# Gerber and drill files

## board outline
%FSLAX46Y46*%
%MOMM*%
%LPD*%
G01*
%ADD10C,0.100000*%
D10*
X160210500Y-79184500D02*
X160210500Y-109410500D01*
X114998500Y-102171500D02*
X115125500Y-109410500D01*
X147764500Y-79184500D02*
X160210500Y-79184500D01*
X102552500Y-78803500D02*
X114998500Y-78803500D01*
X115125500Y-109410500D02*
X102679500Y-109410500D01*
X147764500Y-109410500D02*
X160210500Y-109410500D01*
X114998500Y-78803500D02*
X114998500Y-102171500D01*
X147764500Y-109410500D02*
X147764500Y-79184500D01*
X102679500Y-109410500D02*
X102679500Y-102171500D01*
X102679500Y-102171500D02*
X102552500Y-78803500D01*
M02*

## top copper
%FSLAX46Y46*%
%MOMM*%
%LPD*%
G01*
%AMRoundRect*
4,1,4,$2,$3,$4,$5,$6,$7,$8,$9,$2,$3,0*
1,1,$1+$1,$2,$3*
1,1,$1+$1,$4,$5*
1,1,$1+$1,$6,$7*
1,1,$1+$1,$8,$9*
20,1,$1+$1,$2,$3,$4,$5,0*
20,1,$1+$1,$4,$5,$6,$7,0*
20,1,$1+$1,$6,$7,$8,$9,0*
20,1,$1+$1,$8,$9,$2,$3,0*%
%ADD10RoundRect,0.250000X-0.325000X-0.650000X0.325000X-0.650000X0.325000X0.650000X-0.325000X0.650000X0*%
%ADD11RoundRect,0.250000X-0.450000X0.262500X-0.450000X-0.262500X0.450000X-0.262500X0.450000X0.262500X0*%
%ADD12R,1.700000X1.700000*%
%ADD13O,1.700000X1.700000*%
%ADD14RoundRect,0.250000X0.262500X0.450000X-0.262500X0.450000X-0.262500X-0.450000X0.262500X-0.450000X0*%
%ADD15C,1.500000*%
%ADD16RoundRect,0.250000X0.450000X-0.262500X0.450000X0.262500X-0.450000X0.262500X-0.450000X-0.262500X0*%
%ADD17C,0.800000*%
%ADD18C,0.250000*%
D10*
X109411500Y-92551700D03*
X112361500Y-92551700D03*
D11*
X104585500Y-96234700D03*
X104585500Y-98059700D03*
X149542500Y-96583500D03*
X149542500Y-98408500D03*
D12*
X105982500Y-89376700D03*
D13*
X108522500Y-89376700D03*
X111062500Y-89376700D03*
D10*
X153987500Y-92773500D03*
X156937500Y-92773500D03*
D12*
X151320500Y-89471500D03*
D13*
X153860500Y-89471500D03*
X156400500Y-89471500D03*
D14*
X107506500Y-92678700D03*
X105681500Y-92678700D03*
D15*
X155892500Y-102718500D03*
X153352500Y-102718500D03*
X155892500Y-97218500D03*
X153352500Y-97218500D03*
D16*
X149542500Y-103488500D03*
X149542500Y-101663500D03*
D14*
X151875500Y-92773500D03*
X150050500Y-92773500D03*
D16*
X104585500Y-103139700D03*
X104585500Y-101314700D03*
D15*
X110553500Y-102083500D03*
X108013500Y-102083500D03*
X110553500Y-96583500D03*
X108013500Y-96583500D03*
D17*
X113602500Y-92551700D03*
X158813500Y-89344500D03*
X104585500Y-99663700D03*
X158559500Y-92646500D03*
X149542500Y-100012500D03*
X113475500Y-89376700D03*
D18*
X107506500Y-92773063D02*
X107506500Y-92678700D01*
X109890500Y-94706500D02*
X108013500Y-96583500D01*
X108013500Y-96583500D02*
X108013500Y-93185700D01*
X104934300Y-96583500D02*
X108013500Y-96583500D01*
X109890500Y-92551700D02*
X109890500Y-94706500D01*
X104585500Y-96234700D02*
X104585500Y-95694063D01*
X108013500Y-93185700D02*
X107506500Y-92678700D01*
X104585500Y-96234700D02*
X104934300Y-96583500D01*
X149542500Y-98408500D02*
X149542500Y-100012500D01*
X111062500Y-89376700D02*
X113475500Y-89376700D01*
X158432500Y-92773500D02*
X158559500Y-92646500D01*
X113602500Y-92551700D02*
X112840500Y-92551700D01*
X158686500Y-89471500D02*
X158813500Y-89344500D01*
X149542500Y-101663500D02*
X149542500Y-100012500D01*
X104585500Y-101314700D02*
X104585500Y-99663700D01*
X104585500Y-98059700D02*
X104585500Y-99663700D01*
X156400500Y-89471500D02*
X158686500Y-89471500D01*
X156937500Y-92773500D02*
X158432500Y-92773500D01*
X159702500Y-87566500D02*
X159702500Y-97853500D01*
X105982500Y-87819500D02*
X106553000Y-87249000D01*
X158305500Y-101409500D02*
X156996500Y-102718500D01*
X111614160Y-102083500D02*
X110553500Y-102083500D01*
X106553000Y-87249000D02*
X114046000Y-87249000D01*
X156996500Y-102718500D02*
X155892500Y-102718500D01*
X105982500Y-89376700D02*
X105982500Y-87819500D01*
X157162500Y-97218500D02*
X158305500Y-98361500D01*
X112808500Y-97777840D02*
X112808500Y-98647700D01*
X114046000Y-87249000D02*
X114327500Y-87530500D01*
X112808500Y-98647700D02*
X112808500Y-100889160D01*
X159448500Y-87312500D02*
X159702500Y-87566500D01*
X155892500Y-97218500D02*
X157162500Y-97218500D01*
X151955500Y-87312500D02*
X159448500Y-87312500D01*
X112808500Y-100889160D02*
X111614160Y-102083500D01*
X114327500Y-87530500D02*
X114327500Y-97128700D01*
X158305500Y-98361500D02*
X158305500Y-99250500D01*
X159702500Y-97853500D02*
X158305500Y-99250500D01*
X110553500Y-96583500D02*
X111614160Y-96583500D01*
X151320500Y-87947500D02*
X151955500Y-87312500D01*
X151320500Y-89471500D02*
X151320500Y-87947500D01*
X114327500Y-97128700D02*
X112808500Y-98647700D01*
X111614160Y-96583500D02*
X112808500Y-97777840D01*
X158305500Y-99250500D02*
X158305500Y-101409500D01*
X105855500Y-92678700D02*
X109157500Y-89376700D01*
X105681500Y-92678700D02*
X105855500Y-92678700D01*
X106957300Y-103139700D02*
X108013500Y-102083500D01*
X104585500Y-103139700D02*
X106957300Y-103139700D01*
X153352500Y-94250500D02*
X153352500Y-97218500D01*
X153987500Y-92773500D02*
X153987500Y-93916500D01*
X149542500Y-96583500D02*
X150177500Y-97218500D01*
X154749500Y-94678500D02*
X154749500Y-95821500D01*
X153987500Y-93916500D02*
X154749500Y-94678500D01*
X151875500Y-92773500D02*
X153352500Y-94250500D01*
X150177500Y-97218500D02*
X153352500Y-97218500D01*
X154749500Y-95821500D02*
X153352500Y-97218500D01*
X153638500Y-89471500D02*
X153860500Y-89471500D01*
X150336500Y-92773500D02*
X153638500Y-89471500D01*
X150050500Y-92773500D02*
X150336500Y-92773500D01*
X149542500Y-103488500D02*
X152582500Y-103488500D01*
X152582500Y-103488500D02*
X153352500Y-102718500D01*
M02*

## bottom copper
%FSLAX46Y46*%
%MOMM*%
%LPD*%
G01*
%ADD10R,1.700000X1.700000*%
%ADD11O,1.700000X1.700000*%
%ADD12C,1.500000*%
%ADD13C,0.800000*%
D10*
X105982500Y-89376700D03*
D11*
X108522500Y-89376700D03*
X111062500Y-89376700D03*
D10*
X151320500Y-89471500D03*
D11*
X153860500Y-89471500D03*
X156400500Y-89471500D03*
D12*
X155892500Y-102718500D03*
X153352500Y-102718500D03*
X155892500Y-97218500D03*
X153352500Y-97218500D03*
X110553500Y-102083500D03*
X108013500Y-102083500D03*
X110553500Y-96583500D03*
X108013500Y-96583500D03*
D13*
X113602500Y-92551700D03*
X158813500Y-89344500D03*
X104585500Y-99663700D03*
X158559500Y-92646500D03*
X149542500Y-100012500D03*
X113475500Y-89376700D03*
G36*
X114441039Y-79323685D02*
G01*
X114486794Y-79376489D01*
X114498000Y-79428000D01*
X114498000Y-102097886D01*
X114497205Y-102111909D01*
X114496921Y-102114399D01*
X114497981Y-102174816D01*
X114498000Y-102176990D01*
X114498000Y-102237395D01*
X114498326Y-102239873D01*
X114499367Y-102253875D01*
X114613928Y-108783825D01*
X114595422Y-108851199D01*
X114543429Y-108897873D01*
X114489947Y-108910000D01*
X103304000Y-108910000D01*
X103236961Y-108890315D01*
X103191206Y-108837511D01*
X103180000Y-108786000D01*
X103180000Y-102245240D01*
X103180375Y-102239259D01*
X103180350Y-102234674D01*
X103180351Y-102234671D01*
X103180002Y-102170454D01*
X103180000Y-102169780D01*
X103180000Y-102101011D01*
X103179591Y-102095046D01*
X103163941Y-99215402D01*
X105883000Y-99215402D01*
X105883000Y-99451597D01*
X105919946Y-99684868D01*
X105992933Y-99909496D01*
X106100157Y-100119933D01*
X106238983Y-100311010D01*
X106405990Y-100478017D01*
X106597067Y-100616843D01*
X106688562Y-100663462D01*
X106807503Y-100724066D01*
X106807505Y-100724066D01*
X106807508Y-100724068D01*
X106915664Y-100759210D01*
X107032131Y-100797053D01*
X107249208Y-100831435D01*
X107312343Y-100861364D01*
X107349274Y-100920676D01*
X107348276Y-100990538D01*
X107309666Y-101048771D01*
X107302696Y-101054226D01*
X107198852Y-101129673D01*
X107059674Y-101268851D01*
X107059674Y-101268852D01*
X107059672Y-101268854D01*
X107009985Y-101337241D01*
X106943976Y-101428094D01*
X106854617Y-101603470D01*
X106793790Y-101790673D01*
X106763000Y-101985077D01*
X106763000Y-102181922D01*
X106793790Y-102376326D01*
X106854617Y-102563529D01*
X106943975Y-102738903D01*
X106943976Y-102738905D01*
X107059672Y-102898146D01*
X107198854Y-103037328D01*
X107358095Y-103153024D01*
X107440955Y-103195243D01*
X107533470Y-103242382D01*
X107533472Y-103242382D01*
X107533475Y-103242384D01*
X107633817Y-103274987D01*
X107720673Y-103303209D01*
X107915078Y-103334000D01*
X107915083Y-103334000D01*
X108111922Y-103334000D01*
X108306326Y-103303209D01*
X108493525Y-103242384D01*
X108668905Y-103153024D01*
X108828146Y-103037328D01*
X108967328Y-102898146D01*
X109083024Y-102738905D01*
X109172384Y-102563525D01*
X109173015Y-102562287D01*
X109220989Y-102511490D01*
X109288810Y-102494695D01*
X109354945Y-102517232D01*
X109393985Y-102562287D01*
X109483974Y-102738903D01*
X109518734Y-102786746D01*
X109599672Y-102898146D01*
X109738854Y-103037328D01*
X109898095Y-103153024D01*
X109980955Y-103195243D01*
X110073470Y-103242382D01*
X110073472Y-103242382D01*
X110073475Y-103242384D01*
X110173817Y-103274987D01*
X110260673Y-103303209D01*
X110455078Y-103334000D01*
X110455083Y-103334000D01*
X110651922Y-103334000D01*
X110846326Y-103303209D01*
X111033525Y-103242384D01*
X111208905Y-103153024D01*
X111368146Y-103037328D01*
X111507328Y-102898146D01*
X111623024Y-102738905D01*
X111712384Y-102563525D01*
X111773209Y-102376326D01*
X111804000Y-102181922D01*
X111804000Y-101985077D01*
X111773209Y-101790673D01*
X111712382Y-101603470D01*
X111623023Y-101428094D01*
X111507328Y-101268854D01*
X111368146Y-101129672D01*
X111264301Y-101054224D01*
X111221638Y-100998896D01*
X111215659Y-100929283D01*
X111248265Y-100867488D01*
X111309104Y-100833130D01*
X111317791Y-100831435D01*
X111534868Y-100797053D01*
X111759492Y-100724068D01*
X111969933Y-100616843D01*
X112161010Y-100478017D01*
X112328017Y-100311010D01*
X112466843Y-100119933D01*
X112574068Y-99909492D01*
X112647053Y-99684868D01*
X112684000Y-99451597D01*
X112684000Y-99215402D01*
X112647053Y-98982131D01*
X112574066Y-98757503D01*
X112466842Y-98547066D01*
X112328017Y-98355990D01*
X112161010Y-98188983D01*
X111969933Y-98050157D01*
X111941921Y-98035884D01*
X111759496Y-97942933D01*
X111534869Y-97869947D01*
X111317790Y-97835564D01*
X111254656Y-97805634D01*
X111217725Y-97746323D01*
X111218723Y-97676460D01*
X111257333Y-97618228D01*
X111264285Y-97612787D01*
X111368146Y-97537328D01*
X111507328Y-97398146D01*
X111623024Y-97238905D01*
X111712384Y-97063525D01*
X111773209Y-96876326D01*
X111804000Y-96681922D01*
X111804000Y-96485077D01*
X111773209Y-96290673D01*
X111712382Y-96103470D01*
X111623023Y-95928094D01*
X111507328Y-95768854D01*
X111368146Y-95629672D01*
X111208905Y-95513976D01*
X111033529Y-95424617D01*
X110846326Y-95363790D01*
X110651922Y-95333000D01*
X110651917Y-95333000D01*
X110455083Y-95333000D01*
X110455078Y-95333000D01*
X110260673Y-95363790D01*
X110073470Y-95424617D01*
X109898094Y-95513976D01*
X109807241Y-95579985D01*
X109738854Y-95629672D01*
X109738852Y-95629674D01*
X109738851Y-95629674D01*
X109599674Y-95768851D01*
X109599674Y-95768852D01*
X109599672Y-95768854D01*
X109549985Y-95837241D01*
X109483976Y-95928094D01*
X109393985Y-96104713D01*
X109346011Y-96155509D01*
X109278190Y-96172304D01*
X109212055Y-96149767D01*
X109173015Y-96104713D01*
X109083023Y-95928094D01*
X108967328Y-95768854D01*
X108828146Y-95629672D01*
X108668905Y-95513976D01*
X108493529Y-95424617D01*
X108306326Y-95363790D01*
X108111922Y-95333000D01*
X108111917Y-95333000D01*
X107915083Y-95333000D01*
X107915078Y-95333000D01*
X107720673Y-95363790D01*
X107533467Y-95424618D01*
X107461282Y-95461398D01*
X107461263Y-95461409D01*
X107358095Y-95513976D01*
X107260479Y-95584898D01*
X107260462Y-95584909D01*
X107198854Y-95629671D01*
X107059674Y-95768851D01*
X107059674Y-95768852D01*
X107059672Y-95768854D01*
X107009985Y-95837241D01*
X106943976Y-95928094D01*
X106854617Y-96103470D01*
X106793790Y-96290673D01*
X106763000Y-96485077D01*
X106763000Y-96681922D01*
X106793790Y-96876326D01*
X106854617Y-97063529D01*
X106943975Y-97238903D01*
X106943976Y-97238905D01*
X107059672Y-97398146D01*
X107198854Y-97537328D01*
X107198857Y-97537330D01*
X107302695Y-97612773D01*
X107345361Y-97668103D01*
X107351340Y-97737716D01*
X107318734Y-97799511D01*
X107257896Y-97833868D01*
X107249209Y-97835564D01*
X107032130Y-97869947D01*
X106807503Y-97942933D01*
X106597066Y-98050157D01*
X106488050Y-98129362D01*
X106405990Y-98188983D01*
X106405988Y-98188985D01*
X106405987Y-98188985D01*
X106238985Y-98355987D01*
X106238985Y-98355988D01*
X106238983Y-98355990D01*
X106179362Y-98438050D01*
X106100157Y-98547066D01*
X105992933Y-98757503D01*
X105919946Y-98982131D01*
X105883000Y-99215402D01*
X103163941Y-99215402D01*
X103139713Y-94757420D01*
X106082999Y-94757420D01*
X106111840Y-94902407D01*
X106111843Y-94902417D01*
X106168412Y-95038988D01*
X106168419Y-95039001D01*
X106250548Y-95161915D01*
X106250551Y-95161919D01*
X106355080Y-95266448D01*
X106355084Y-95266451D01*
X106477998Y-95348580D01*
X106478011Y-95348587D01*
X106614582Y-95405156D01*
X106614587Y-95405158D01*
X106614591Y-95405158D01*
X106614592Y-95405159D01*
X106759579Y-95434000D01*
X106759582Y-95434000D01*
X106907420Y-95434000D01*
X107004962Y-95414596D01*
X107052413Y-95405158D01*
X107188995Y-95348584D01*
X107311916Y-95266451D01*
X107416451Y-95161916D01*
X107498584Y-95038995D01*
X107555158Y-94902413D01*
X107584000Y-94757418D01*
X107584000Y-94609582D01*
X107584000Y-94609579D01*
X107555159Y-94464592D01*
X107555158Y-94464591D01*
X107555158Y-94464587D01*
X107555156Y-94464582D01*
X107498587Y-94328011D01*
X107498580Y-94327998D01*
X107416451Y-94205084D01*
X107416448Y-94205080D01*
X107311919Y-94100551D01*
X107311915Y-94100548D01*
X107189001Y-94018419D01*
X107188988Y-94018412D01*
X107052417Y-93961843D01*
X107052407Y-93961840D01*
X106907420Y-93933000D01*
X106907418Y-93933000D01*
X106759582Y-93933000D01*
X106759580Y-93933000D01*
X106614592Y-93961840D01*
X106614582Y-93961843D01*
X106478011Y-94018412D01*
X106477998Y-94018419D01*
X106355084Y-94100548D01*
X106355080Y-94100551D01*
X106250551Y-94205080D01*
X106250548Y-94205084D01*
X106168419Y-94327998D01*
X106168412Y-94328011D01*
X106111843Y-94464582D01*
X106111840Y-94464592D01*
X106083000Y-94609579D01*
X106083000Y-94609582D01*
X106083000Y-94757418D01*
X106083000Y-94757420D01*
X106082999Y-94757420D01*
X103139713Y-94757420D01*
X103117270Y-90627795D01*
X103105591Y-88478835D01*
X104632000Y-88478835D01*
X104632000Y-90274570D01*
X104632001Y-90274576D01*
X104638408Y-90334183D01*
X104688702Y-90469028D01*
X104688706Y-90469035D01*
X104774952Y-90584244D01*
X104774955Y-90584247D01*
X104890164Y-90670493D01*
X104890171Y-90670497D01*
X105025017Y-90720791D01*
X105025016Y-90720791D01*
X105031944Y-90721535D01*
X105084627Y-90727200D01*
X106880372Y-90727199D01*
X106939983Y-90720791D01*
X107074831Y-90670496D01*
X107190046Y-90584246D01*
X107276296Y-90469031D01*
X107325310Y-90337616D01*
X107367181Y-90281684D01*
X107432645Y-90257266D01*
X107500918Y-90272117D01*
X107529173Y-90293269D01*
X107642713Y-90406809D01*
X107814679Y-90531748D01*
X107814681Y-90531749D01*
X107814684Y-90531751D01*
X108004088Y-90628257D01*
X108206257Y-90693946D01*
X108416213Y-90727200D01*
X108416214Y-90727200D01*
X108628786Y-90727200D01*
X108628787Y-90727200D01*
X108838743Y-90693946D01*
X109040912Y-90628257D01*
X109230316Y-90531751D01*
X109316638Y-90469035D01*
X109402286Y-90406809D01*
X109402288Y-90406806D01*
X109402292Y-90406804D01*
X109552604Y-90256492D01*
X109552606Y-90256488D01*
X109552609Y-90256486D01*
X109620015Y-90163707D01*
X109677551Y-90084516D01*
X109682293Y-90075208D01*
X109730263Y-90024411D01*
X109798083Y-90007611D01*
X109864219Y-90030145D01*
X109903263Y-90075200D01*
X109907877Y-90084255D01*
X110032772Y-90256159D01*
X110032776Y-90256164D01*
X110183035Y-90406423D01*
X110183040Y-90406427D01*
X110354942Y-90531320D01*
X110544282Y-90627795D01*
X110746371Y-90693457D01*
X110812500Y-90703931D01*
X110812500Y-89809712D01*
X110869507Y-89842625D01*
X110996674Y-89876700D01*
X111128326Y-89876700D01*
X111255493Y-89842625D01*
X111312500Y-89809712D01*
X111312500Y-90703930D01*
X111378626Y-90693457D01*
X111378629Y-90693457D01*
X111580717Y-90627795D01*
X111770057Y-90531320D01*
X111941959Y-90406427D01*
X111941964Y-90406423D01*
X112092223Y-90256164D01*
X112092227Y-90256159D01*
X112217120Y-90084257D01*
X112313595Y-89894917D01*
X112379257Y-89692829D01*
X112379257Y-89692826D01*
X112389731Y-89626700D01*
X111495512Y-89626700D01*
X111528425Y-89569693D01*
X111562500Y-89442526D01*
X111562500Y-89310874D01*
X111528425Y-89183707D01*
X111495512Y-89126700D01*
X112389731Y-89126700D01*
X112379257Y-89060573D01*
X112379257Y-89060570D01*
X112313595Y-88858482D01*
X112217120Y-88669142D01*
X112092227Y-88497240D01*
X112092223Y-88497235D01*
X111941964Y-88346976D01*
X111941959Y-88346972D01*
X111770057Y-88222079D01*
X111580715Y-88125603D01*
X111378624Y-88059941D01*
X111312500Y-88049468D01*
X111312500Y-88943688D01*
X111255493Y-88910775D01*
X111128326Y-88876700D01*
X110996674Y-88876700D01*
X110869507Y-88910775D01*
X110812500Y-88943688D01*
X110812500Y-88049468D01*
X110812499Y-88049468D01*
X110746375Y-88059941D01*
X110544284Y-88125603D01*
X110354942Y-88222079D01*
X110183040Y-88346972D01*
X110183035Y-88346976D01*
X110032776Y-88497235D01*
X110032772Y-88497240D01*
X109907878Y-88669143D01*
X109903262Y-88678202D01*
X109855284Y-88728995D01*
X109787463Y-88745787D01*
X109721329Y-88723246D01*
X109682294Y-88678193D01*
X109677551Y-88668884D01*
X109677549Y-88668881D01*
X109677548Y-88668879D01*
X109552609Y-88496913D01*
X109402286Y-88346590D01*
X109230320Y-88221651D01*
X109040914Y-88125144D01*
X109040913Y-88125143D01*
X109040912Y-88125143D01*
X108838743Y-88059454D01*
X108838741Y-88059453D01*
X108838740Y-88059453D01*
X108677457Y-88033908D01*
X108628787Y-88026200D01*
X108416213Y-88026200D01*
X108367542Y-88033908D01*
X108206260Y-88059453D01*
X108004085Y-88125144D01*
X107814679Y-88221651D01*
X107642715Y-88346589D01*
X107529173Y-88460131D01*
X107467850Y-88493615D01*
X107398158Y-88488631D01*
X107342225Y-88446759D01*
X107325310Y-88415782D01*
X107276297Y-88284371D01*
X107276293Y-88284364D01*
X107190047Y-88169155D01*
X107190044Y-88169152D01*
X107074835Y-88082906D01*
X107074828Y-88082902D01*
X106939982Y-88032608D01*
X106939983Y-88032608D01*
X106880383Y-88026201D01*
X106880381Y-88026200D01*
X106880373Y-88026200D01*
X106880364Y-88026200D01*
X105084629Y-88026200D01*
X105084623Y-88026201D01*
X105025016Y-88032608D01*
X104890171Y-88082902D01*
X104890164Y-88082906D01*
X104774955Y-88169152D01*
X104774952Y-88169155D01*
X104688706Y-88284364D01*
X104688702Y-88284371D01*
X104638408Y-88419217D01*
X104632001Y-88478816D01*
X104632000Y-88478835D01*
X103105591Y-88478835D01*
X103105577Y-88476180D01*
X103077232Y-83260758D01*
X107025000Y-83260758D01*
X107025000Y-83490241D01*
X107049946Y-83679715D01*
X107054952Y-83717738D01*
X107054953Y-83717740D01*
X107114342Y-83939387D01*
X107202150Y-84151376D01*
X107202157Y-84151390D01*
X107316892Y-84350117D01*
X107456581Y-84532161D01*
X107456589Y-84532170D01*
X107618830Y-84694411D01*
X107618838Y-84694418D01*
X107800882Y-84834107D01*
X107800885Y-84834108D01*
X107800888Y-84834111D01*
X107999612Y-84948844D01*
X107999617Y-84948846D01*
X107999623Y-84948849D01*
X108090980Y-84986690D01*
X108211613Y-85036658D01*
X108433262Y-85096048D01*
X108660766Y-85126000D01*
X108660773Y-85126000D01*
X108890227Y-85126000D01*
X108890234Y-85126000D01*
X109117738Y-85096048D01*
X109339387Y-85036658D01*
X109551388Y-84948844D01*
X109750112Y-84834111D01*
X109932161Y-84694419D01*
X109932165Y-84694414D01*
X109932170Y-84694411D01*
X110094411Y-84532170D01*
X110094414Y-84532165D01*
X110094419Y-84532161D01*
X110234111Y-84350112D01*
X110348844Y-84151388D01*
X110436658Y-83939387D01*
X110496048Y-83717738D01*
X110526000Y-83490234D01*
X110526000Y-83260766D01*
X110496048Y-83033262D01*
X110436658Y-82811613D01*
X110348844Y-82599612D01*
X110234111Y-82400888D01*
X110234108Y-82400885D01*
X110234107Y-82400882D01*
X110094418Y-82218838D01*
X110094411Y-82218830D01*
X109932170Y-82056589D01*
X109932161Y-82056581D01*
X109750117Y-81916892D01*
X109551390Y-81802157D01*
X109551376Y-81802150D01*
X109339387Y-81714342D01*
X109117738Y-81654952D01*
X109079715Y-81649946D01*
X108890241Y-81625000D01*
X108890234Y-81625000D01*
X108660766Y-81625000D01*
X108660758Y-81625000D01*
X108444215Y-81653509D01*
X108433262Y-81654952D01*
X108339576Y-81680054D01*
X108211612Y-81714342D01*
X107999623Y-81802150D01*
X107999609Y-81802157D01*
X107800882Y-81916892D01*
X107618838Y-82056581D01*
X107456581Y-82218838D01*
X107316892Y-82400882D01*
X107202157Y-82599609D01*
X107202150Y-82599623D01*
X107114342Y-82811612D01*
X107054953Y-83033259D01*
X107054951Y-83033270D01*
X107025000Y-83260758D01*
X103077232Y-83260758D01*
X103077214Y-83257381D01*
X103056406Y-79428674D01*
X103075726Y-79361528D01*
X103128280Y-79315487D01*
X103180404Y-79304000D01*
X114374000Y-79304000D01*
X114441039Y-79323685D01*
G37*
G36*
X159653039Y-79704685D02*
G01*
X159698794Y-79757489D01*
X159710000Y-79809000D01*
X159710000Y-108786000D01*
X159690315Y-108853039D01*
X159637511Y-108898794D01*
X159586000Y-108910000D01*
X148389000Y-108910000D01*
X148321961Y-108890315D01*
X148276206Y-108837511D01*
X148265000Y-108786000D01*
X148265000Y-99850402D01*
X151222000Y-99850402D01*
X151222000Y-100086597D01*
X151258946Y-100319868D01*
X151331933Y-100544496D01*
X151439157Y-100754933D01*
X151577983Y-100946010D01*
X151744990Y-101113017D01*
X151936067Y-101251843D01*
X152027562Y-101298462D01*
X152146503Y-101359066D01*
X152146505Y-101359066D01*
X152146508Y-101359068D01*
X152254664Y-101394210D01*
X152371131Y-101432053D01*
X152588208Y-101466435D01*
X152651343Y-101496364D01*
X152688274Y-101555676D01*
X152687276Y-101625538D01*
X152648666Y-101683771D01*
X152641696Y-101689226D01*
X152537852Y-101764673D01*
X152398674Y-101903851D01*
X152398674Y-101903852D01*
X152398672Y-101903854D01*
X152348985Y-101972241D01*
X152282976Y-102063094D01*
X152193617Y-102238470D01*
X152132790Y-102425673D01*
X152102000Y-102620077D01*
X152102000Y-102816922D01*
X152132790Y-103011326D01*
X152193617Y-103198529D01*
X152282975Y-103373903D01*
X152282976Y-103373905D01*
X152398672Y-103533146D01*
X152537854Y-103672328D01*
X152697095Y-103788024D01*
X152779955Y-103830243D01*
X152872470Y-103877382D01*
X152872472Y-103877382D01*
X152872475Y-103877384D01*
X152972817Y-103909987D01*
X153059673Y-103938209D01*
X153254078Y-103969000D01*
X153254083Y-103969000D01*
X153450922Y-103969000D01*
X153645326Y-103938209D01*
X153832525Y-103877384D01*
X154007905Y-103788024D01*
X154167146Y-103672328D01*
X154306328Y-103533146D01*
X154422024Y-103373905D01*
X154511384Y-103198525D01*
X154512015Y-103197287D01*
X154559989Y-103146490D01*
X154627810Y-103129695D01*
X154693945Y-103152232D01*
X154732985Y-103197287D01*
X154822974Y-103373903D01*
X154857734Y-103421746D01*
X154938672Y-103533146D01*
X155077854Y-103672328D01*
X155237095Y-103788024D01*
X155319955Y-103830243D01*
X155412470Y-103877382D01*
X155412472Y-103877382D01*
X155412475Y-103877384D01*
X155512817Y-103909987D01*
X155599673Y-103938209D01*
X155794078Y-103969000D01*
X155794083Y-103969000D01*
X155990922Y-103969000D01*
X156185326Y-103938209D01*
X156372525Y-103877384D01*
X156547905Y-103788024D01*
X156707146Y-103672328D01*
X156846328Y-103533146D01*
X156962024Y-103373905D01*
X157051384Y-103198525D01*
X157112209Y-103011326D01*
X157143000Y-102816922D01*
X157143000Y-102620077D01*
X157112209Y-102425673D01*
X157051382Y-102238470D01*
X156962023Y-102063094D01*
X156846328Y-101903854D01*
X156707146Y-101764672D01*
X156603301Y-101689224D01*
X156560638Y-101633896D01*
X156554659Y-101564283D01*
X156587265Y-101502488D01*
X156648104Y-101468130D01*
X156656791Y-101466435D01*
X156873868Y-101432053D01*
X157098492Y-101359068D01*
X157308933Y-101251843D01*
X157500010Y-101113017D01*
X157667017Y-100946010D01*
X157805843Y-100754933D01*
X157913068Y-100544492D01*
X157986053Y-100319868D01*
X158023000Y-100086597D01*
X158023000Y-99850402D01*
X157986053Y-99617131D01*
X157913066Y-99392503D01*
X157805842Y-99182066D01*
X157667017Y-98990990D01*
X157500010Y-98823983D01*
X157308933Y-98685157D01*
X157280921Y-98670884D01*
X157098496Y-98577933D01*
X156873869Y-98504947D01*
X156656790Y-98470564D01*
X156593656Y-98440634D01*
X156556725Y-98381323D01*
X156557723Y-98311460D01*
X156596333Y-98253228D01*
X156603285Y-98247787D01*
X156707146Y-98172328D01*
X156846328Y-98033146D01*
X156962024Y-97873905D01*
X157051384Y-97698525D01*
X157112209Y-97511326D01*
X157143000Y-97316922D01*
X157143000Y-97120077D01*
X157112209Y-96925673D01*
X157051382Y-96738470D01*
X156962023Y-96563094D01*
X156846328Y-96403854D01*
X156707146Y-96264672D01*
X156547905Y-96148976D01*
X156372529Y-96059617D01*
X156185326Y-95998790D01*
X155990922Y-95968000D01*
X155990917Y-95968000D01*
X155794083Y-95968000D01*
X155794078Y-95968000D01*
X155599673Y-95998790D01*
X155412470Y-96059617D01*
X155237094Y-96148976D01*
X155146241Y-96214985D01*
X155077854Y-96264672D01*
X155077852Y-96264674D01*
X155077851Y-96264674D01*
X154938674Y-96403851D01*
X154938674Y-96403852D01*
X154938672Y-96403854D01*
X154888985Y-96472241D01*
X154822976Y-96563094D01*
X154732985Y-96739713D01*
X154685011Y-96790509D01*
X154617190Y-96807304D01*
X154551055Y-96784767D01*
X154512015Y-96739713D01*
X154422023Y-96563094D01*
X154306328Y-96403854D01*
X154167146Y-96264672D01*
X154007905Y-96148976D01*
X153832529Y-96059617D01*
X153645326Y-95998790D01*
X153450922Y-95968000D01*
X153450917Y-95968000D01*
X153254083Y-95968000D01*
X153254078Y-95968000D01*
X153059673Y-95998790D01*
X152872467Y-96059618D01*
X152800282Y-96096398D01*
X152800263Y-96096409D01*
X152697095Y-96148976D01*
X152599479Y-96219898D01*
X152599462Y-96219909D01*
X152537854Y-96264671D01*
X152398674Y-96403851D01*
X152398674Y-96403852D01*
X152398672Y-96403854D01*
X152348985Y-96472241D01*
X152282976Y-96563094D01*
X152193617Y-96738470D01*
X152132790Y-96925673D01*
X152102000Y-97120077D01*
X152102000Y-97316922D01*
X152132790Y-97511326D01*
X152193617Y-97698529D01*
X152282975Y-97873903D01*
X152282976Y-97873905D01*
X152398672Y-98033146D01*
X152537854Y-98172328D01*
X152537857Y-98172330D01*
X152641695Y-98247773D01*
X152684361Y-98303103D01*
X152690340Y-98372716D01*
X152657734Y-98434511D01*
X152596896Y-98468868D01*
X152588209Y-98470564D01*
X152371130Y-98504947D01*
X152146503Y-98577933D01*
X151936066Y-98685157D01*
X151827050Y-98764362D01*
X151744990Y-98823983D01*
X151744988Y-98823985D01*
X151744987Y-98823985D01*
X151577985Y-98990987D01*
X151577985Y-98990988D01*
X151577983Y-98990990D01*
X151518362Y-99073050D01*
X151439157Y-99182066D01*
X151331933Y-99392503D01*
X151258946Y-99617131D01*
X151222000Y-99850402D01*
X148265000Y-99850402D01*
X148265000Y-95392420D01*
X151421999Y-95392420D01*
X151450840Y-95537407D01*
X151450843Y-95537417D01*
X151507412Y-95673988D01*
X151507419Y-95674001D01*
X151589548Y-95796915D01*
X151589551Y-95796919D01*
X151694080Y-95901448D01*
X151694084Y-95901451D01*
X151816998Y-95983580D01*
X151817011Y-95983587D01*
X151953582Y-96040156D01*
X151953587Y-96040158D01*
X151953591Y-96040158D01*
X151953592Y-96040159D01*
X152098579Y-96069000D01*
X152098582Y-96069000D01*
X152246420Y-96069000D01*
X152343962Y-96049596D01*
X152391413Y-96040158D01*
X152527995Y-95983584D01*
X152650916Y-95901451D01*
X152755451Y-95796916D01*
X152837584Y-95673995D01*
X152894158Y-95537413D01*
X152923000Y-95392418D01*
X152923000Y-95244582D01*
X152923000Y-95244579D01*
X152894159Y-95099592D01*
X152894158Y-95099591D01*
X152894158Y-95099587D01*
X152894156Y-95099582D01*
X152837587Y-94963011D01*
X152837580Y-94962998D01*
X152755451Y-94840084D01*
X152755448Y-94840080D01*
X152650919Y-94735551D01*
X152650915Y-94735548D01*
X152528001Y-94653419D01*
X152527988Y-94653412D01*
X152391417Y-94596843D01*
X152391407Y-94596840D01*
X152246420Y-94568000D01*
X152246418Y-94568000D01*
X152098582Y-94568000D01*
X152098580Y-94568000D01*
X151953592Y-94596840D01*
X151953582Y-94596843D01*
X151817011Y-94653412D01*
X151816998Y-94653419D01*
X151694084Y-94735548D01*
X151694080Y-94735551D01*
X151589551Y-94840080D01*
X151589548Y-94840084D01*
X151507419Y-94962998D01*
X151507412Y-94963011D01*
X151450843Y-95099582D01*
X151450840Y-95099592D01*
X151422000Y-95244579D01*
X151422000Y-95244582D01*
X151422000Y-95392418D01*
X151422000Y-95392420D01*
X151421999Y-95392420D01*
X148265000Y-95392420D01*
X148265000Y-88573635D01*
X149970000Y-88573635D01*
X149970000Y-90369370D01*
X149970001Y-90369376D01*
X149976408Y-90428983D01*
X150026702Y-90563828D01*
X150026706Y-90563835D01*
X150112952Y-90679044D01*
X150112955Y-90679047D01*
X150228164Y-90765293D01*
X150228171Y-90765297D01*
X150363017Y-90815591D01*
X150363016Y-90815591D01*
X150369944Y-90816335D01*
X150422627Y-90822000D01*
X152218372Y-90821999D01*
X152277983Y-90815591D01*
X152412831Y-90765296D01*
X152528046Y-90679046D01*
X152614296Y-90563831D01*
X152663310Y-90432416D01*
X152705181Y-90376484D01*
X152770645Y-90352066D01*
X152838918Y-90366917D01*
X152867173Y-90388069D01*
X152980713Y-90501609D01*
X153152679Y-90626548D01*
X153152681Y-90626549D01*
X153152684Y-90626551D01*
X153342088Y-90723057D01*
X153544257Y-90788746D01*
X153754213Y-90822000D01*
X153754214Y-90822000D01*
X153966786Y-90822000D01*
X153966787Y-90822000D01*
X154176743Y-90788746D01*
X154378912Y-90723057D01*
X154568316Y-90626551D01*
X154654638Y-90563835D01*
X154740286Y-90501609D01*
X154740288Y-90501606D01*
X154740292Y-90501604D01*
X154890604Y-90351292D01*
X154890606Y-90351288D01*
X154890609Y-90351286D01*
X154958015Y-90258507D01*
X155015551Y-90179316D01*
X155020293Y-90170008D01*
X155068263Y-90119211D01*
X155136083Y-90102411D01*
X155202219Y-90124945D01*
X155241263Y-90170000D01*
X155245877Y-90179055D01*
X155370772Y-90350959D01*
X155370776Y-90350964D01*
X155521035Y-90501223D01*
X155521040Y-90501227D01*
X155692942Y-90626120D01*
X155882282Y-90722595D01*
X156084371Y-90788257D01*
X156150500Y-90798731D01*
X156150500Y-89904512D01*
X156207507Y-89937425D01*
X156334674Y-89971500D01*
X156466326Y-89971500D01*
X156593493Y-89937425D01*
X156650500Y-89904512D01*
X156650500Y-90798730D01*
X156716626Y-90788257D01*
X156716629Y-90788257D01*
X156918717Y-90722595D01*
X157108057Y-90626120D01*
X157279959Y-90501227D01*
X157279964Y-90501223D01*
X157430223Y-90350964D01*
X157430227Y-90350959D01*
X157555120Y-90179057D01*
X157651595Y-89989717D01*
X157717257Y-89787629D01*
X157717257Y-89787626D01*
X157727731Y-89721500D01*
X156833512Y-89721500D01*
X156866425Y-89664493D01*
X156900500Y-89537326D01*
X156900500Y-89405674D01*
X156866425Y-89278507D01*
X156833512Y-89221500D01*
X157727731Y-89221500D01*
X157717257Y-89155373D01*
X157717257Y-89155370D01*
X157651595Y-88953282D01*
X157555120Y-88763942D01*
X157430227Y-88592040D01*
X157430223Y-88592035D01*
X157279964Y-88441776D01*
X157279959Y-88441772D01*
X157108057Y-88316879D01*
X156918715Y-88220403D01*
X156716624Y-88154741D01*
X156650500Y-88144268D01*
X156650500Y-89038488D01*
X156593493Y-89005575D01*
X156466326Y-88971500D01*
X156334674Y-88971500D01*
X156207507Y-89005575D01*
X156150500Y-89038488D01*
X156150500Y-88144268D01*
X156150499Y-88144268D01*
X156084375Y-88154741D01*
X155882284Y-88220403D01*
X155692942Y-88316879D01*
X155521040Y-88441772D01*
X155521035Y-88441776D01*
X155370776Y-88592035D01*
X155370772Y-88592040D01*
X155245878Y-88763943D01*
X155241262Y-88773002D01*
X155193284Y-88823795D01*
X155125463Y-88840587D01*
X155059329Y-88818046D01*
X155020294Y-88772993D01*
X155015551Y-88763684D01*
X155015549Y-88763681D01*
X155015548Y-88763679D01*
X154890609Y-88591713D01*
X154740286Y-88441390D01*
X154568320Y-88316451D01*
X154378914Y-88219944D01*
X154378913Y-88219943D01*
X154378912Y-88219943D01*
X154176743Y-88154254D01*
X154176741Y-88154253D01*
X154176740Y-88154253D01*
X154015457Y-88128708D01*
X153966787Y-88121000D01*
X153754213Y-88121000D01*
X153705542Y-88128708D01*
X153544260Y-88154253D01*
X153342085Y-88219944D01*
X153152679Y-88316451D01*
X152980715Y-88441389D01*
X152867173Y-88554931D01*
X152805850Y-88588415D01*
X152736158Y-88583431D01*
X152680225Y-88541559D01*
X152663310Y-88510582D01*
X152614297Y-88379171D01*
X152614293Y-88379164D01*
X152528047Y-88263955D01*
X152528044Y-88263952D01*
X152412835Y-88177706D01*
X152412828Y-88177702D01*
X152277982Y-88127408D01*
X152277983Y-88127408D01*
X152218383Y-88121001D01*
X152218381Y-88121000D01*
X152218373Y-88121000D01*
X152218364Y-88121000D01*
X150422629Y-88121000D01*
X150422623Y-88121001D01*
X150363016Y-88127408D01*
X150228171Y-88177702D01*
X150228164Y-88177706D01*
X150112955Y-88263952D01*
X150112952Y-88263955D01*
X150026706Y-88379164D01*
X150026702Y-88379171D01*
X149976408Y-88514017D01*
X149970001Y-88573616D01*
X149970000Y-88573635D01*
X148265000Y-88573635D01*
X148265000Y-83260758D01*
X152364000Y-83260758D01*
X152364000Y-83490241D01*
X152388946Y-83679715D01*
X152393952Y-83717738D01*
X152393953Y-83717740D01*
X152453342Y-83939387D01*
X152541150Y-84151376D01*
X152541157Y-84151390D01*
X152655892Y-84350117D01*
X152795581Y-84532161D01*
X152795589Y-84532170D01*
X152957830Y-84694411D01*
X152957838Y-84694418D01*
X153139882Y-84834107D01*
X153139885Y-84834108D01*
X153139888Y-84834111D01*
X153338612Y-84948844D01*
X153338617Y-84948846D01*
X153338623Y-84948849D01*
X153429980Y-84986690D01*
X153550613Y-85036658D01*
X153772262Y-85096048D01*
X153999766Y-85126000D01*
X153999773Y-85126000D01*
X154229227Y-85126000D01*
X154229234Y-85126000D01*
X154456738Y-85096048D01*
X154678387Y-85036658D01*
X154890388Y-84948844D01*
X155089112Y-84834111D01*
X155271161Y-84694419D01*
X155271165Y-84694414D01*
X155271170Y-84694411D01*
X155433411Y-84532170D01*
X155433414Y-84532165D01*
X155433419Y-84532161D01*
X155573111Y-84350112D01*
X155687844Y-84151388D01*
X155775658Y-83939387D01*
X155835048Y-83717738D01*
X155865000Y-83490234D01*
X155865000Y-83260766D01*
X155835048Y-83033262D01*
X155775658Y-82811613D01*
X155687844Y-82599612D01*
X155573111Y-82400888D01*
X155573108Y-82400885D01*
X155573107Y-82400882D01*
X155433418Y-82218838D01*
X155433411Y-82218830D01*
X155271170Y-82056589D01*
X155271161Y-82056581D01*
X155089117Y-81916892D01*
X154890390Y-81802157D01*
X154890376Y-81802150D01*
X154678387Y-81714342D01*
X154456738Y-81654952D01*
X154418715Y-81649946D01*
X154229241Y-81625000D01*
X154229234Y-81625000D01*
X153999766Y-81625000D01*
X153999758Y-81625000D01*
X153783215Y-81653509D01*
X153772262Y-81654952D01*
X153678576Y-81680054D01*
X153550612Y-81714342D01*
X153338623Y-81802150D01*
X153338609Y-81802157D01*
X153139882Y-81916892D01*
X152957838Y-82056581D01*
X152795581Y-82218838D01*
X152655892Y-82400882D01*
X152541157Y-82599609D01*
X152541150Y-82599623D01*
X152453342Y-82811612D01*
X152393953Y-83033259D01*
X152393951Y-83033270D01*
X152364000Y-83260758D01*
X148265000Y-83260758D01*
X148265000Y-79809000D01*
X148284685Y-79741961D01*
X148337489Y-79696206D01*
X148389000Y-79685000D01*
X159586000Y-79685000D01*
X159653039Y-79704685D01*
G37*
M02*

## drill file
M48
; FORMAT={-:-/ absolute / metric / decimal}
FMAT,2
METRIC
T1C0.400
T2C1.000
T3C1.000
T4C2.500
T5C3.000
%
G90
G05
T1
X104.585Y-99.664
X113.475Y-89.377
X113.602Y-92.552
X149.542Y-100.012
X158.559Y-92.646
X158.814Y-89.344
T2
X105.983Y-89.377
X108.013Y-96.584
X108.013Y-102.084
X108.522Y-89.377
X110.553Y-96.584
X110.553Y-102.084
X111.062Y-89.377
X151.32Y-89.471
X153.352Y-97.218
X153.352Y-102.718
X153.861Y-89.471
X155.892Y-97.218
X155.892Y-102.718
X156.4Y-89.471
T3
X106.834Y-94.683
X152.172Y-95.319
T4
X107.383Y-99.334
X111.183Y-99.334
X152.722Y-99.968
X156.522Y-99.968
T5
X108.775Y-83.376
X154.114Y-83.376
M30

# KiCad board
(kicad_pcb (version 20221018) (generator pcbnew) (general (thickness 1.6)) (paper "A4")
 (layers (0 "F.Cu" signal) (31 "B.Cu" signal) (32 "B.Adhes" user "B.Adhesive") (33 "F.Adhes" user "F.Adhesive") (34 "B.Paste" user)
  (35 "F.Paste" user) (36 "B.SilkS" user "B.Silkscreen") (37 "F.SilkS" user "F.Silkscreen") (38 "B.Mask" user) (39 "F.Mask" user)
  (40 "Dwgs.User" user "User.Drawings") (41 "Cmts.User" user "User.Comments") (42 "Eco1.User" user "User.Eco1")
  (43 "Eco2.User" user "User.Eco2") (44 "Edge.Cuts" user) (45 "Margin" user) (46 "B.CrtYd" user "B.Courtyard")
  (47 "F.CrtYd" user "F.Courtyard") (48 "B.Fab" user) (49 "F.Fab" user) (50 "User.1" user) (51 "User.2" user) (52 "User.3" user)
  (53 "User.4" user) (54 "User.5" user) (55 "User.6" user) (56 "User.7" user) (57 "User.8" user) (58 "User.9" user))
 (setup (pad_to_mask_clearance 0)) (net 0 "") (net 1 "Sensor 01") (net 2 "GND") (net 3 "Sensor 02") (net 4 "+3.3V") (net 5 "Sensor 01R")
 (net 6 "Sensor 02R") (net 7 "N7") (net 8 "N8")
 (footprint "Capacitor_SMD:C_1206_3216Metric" (layer "F.Cu") (at 110.8865 92.5517)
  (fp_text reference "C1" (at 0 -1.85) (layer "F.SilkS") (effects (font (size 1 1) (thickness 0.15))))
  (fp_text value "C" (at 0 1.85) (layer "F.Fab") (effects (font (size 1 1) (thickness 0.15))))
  (pad "1" smd roundrect (at -1.475 0) (size 1.15 1.8) (layers "F.Cu" "F.Paste" "F.Mask") (roundrect_rratio 0.217391) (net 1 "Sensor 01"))
  (pad "2" smd roundrect (at 1.475 0) (size 1.15 1.8) (layers "F.Cu" "F.Paste" "F.Mask") (roundrect_rratio 0.217391) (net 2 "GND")))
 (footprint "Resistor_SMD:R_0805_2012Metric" (layer "F.Cu") (at 104.5855 97.1472 -90)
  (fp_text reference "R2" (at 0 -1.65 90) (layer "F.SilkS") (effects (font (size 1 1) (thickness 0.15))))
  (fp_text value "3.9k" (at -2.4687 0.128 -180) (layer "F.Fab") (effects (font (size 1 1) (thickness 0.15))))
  (pad "1" smd roundrect (at -0.9125 0 270) (size 1.025 1.4) (layers "F.Cu" "F.Paste" "F.Mask") (roundrect_rratio 0.243902)
   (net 1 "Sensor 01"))
  (pad "2" smd roundrect (at 0.9125 0 270) (size 1.025 1.4) (layers "F.Cu" "F.Paste" "F.Mask") (roundrect_rratio 0.243902) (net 2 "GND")))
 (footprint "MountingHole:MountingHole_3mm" (layer "F.Cu") (at 108.7755 83.3755)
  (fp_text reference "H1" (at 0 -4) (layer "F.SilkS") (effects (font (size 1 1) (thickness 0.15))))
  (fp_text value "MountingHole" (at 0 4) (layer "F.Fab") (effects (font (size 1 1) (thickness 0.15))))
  (pad "" np_thru_hole circle (at 0 0) (size 3 3) (drill 3) (layers "*.Cu" "*.Mask")))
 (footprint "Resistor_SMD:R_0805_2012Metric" (layer "F.Cu") (at 149.5425 97.496 -90)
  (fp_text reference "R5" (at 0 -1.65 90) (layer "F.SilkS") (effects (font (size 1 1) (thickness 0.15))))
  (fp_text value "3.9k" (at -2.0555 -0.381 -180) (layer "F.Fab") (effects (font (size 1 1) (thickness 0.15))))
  (pad "1" smd roundrect (at -0.9125 0 270) (size 1.025 1.4) (layers "F.Cu" "F.Paste" "F.Mask") (roundrect_rratio 0.243902)
   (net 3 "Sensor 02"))
  (pad "2" smd roundrect (at 0.9125 0 270) (size 1.025 1.4) (layers "F.Cu" "F.Paste" "F.Mask") (roundrect_rratio 0.243902) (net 2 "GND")))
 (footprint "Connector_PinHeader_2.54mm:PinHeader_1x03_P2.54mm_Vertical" (layer "F.Cu") (at 105.9825 89.3767 90)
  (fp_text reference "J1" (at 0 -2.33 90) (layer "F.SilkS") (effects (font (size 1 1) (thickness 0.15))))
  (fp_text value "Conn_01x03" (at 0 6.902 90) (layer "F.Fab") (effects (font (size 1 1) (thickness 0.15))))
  (pad "1" thru_hole rect (at 0 0 90) (size 1.7 1.7) (drill 1) (layers "*.Cu" "*.Mask") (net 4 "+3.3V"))
  (pad "2" thru_hole oval (at 0 2.54 90) (size 1.7 1.7) (drill 1) (layers "*.Cu" "*.Mask") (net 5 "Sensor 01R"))
  (pad "3" thru_hole oval (at 0 5.08 90) (size 1.7 1.7) (drill 1) (layers "*.Cu" "*.Mask") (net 2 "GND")))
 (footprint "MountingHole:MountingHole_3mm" (layer "F.Cu") (at 154.1145 83.3755)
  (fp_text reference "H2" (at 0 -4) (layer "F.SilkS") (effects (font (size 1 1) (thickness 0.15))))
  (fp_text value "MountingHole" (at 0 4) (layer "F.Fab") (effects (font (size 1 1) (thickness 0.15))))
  (pad "" np_thru_hole circle (at 0 0) (size 3 3) (drill 3) (layers "*.Cu" "*.Mask")))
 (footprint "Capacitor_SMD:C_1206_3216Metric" (layer "F.Cu") (at 155.4625 92.7735)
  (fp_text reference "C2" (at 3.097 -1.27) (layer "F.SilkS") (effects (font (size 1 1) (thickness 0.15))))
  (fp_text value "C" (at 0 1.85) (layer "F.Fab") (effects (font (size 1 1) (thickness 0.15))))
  (pad "1" smd roundrect (at -1.475 0) (size 1.15 1.8) (layers "F.Cu" "F.Paste" "F.Mask") (roundrect_rratio 0.217391) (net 3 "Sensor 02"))
  (pad "2" smd roundrect (at 1.475 0) (size 1.15 1.8) (layers "F.Cu" "F.Paste" "F.Mask") (roundrect_rratio 0.217391) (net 2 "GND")))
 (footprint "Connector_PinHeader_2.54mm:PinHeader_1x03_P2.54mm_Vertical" (layer "F.Cu") (at 151.3205 89.4715 90)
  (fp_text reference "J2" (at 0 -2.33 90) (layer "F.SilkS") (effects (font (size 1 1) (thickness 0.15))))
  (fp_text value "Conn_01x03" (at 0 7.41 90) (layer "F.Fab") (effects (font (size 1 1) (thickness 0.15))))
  (pad "1" thru_hole rect (at 0 0 90) (size 1.7 1.7) (drill 1) (layers "*.Cu" "*.Mask") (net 4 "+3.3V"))
  (pad "2" thru_hole oval (at 0 2.54 90) (size 1.7 1.7) (drill 1) (layers "*.Cu" "*.Mask") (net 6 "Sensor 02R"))
  (pad "3" thru_hole oval (at 0 5.08 90) (size 1.7 1.7) (drill 1) (layers "*.Cu" "*.Mask") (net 2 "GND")))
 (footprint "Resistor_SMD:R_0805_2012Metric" (layer "F.Cu") (at 106.594 92.6787 180)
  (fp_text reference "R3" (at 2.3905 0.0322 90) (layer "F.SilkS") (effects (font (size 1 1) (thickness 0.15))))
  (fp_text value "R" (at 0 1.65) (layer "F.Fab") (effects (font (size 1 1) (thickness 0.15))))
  (pad "1" smd roundrect (at -0.9125 0 180) (size 1.025 1.4) (layers "F.Cu" "F.Paste" "F.Mask") (roundrect_rratio 0.243902)
   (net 1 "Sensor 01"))
  (pad "2" smd roundrect (at 0.9125 0 180) (size 1.025 1.4) (layers "F.Cu" "F.Paste" "F.Mask") (roundrect_rratio 0.243902)
   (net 5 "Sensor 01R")))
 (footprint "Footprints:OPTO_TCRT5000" (layer "F.Cu") (at 154.6225 99.9685 -90)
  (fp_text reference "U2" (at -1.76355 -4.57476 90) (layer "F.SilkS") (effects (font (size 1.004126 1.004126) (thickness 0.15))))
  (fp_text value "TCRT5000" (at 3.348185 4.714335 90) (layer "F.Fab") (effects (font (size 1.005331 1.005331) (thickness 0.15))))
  (pad "" np_thru_hole circle (at -4.65 2.45 270) (size 1 1) (drill 1) (layers "*.Cu" "*.Mask"))
  (pad "" np_thru_hole circle (at 0 -1.9 270) (size 2.5 2.5) (drill 2.5) (layers "*.Cu" "*.Mask"))
  (pad "" np_thru_hole circle (at 0 1.9 270) (size 2.5 2.5) (drill 2.5) (layers "*.Cu" "*.Mask"))
  (pad "A" thru_hole circle (at 2.75 -1.27 270) (size 1.5 1.5) (drill 1) (layers "*.Cu" "*.Mask") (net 4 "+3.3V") (solder_mask_margin 0.102))
  (pad "CATH" thru_hole circle (at 2.75 1.27 270) (size 1.5 1.5) (drill 1) (layers "*.Cu" "*.Mask") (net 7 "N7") (solder_mask_margin 0.102))
  (pad "COLL" thru_hole circle (at -2.75 -1.27 270) (size 1.5 1.5) (drill 1) (layers "*.Cu" "*.Mask") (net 4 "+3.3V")
   (solder_mask_margin 0.102))
  (pad "E" thru_hole circle (at -2.75 1.27 270) (size 1.5 1.5) (drill 1) (layers "*.Cu" "*.Mask") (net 3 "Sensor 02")
   (solder_mask_margin 0.102)))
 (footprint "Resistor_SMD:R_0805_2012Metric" (layer "F.Cu") (at 149.5425 102.576 90)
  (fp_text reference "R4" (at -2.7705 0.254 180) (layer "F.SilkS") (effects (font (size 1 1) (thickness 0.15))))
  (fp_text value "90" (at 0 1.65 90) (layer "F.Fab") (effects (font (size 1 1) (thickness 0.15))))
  (pad "1" smd roundrect (at -0.9125 0 90) (size 1.025 1.4) (layers "F.Cu" "F.Paste" "F.Mask") (roundrect_rratio 0.243902) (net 7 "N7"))
  (pad "2" smd roundrect (at 0.9125 0 90) (size 1.025 1.4) (layers "F.Cu" "F.Paste" "F.Mask") (roundrect_rratio 0.243902) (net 2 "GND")))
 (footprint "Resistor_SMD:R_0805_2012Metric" (layer "F.Cu") (at 150.963 92.7735 180)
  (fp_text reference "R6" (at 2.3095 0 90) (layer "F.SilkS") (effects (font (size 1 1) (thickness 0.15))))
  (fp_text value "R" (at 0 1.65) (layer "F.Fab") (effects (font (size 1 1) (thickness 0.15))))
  (pad "1" smd roundrect (at -0.9125 0 180) (size 1.025 1.4) (layers "F.Cu" "F.Paste" "F.Mask") (roundrect_rratio 0.243902)
   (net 3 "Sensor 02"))
  (pad "2" smd roundrect (at 0.9125 0 180) (size 1.025 1.4) (layers "F.Cu" "F.Paste" "F.Mask") (roundrect_rratio 0.243902)
   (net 6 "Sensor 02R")))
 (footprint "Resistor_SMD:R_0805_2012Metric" (layer "F.Cu") (at 104.5855 102.2272 90)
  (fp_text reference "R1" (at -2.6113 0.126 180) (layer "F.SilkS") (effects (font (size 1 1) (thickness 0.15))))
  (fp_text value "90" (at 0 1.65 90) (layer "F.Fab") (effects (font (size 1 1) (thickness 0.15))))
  (pad "1" smd roundrect (at -0.9125 0 90) (size 1.025 1.4) (layers "F.Cu" "F.Paste" "F.Mask") (roundrect_rratio 0.243902) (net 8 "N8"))
  (pad "2" smd roundrect (at 0.9125 0 90) (size 1.025 1.4) (layers "F.Cu" "F.Paste" "F.Mask") (roundrect_rratio 0.243902) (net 2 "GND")))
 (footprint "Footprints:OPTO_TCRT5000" (layer "F.Cu") (at 109.2835 99.3335 -90)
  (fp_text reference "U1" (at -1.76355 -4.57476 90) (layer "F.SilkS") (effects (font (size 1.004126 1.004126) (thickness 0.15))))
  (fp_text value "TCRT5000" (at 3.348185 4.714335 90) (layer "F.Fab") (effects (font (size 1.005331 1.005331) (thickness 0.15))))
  (pad "" np_thru_hole circle (at -4.65 2.45 270) (size 1 1) (drill 1) (layers "*.Cu" "*.Mask"))
  (pad "" np_thru_hole circle (at 0 -1.9 270) (size 2.5 2.5) (drill 2.5) (layers "*.Cu" "*.Mask"))
  (pad "" np_thru_hole circle (at 0 1.9 270) (size 2.5 2.5) (drill 2.5) (layers "*.Cu" "*.Mask"))
  (pad "A" thru_hole circle (at 2.75 -1.27 270) (size 1.5 1.5) (drill 1) (layers "*.Cu" "*.Mask") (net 4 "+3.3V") (solder_mask_margin 0.102))
  (pad "CATH" thru_hole circle (at 2.75 1.27 270) (size 1.5 1.5) (drill 1) (layers "*.Cu" "*.Mask") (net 8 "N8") (solder_mask_margin 0.102))
  (pad "COLL" thru_hole circle (at -2.75 -1.27 270) (size 1.5 1.5) (drill 1) (layers "*.Cu" "*.Mask") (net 4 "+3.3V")
   (solder_mask_margin 0.102))
  (pad "E" thru_hole circle (at -2.75 1.27 270) (size 1.5 1.5) (drill 1) (layers "*.Cu" "*.Mask") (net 1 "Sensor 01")
   (solder_mask_margin 0.102)))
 (gr_line (start 160.2105 79.1845) (end 160.2105 109.4105) (stroke (width 0.1) (type default)) (layer "Edge.Cuts"))
 (gr_line (start 114.9985 102.1715) (end 115.1255 109.4105) (stroke (width 0.1) (type default)) (layer "Edge.Cuts"))
 (gr_line (start 147.7645 79.1845) (end 160.2105 79.1845) (stroke (width 0.1) (type default)) (layer "Edge.Cuts"))
 (gr_line (start 102.5525 78.8035) (end 114.9985 78.8035) (stroke (width 0.1) (type default)) (layer "Edge.Cuts"))
 (gr_line (start 115.1255 109.4105) (end 102.6795 109.4105) (stroke (width 0.1) (type default)) (layer "Edge.Cuts"))
 (gr_line (start 147.7645 109.4105) (end 160.2105 109.4105) (stroke (width 0.1) (type default)) (layer "Edge.Cuts"))
 (gr_line (start 114.9985 78.8035) (end 114.9985 102.1715) (stroke (width 0.1) (type default)) (layer "Edge.Cuts"))
 (gr_line (start 147.7645 109.4105) (end 147.7645 79.1845) (stroke (width 0.1) (type default)) (layer "Edge.Cuts"))
 (gr_line (start 102.6795 109.4105) (end 102.6795 102.1715) (stroke (width 0.1) (type default)) (layer "Edge.Cuts"))
 (gr_line (start 102.6795 102.1715) (end 102.5525 78.8035) (stroke (width 0.1) (type default)) (layer "Edge.Cuts"))
 (segment (start 107.5065 92.773063) (end 107.5065 92.6787) (width 0.25) (layer "F.Cu") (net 1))
 (segment (start 109.8905 94.7065) (end 108.0135 96.5835) (width 0.25) (layer "F.Cu") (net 1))
 (segment (start 108.0135 96.5835) (end 108.0135 93.1857) (width 0.25) (layer "F.Cu") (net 1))
 (segment (start 104.9343 96.5835) (end 108.0135 96.5835) (width 0.25) (layer "F.Cu") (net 1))
 (segment (start 109.8905 92.5517) (end 109.8905 94.7065) (width 0.25) (layer "F.Cu") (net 1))
 (segment (start 104.5855 96.2347) (end 104.5855 95.694063) (width 0.25) (layer "F.Cu") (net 1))
 (segment (start 108.0135 93.1857) (end 107.5065 92.6787) (width 0.25) (layer "F.Cu") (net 1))
 (segment (start 104.5855 96.2347) (end 104.9343 96.5835) (width 0.25) (layer "F.Cu") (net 1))
 (segment (start 149.5425 98.4085) (end 149.5425 100.0125) (width 0.25) (layer "F.Cu") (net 2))
 (segment (start 111.0625 89.3767) (end 113.4755 89.3767) (width 0.25) (layer "F.Cu") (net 2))
 (segment (start 158.4325 92.7735) (end 158.5595 92.6465) (width 0.25) (layer "F.Cu") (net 2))
 (segment (start 113.6025 92.5517) (end 112.8405 92.5517) (width 0.25) (layer "F.Cu") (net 2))
 (segment (start 158.6865 89.4715) (end 158.8135 89.3445) (width 0.25) (layer "F.Cu") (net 2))
 (segment (start 149.5425 101.6635) (end 149.5425 100.0125) (width 0.25) (layer "F.Cu") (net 2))
 (segment (start 104.5855 101.3147) (end 104.5855 99.6637) (width 0.25) (layer "F.Cu") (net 2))
 (segment (start 104.5855 98.0597) (end 104.5855 99.6637) (width 0.25) (layer "F.Cu") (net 2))
 (segment (start 156.4005 89.4715) (end 158.6865 89.4715) (width 0.25) (layer "F.Cu") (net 2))
 (segment (start 156.9375 92.7735) (end 158.4325 92.7735) (width 0.25) (layer "F.Cu") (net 2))
 (via (at 113.6025 92.5517) (size 0.8) (drill 0.4) (layers "F.Cu" "B.Cu") (free) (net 2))
 (via (at 158.8135 89.3445) (size 0.8) (drill 0.4) (layers "F.Cu" "B.Cu") (free) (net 2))
 (via (at 104.5855 99.6637) (size 0.8) (drill 0.4) (layers "F.Cu" "B.Cu") (free) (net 2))
 (via (at 158.5595 92.6465) (size 0.8) (drill 0.4) (layers "F.Cu" "B.Cu") (free) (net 2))
 (via (at 149.5425 100.0125) (size 0.8) (drill 0.4) (layers "F.Cu" "B.Cu") (free) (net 2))
 (via (at 113.4755 89.3767) (size 0.8) (drill 0.4) (layers "F.Cu" "B.Cu") (free) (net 2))
 (segment (start 159.7025 87.5665) (end 159.7025 97.8535) (width 0.25) (layer "F.Cu") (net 4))
 (segment (start 105.9825 87.8195) (end 106.553 87.249) (width 0.25) (layer "F.Cu") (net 4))
 (segment (start 158.3055 101.4095) (end 156.9965 102.7185) (width 0.25) (layer "F.Cu") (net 4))
 (segment (start 111.61416 102.0835) (end 110.5535 102.0835) (width 0.25) (layer "F.Cu") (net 4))
 (segment (start 106.553 87.249) (end 114.046 87.249) (width 0.25) (layer "F.Cu") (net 4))
 (segment (start 156.9965 102.7185) (end 155.8925 102.7185) (width 0.25) (layer "F.Cu") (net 4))
 (segment (start 105.9825 89.3767) (end 105.9825 87.8195) (width 0.25) (layer "F.Cu") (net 4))
 (segment (start 157.1625 97.2185) (end 158.3055 98.3615) (width 0.25) (layer "F.Cu") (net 4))
 (segment (start 112.8085 97.77784) (end 112.8085 98.6477) (width 0.25) (layer "F.Cu") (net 4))
 (segment (start 114.046 87.249) (end 114.3275 87.5305) (width 0.25) (layer "F.Cu") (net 4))
 (segment (start 112.8085 98.6477) (end 112.8085 100.88916) (width 0.25) (layer "F.Cu") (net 4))
 (segment (start 159.4485 87.3125) (end 159.7025 87.5665) (width 0.25) (layer "F.Cu") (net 4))
 (segment (start 155.8925 97.2185) (end 157.1625 97.2185) (width 0.25) (layer "F.Cu") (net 4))
 (segment (start 151.9555 87.3125) (end 159.4485 87.3125) (width 0.25) (layer "F.Cu") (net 4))
 (segment (start 112.8085 100.88916) (end 111.61416 102.0835) (width 0.25) (layer "F.Cu") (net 4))
 (segment (start 114.3275 87.5305) (end 114.3275 97.1287) (width 0.25) (layer "F.Cu") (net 4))
 (segment (start 158.3055 98.3615) (end 158.3055 99.2505) (width 0.25) (layer "F.Cu") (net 4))
 (segment (start 159.7025 97.8535) (end 158.3055 99.2505) (width 0.25) (layer "F.Cu") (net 4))
 (segment (start 110.5535 96.5835) (end 111.61416 96.5835) (width 0.25) (layer "F.Cu") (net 4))
 (segment (start 151.3205 87.9475) (end 151.9555 87.3125) (width 0.25) (layer "F.Cu") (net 4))
 (segment (start 151.3205 89.4715) (end 151.3205 87.9475) (width 0.25) (layer "F.Cu") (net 4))
 (segment (start 114.3275 97.1287) (end 112.8085 98.6477) (width 0.25) (layer "F.Cu") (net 4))
 (segment (start 111.61416 96.5835) (end 112.8085 97.77784) (width 0.25) (layer "F.Cu") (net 4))
 (segment (start 158.3055 99.2505) (end 158.3055 101.4095) (width 0.25) (layer "F.Cu") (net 4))
 (segment (start 105.8555 92.6787) (end 109.1575 89.3767) (width 0.25) (layer "F.Cu") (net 5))
 (segment (start 105.6815 92.6787) (end 105.8555 92.6787) (width 0.25) (layer "F.Cu") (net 5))
 (segment (start 106.9573 103.1397) (end 108.0135 102.0835) (width 0.25) (layer "F.Cu") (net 8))
 (segment (start 104.5855 103.1397) (end 106.9573 103.1397) (width 0.25) (layer "F.Cu") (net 8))
 (segment (start 153.3525 94.2505) (end 153.3525 97.2185) (width 0.25) (layer "F.Cu") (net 3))
 (segment (start 153.9875 92.7735) (end 153.9875 93.9165) (width 0.25) (layer "F.Cu") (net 3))
 (segment (start 149.5425 96.5835) (end 150.1775 97.2185) (width 0.25) (layer "F.Cu") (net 3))
 (segment (start 154.7495 94.6785) (end 154.7495 95.8215) (width 0.25) (layer "F.Cu") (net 3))
 (segment (start 153.9875 93.9165) (end 154.7495 94.6785) (width 0.25) (layer "F.Cu") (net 3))
 (segment (start 151.8755 92.7735) (end 153.3525 94.2505) (width 0.25) (layer "F.Cu") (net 3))
 (segment (start 150.1775 97.2185) (end 153.3525 97.2185) (width 0.25) (layer "F.Cu") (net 3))
 (segment (start 154.7495 95.8215) (end 153.3525 97.2185) (width 0.25) (layer "F.Cu") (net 3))
 (segment (start 153.6385 89.4715) (end 153.8605 89.4715) (width 0.25) (layer "F.Cu") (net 6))
 (segment (start 150.3365 92.7735) (end 153.6385 89.4715) (width 0.25) (layer "F.Cu") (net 6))
 (segment (start 150.0505 92.7735) (end 150.3365 92.7735) (width 0.25) (layer "F.Cu") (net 6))
 (segment (start 149.5425 103.4885) (end 152.5825 103.4885) (width 0.25) (layer "F.Cu") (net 7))
 (segment (start 152.5825 103.4885) (end 153.3525 102.7185) (width 0.25) (layer "F.Cu") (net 7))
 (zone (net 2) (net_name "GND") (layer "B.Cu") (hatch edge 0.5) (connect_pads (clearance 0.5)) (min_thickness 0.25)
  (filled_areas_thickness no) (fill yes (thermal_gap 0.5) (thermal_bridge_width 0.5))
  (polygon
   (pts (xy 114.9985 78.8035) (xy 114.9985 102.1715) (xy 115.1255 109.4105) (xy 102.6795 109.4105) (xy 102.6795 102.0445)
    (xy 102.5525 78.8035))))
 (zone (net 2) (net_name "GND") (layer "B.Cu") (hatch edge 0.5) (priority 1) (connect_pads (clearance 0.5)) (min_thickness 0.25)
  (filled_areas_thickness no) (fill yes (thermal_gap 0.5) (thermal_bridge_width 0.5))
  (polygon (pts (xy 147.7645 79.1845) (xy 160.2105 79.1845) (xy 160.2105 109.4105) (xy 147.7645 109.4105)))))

